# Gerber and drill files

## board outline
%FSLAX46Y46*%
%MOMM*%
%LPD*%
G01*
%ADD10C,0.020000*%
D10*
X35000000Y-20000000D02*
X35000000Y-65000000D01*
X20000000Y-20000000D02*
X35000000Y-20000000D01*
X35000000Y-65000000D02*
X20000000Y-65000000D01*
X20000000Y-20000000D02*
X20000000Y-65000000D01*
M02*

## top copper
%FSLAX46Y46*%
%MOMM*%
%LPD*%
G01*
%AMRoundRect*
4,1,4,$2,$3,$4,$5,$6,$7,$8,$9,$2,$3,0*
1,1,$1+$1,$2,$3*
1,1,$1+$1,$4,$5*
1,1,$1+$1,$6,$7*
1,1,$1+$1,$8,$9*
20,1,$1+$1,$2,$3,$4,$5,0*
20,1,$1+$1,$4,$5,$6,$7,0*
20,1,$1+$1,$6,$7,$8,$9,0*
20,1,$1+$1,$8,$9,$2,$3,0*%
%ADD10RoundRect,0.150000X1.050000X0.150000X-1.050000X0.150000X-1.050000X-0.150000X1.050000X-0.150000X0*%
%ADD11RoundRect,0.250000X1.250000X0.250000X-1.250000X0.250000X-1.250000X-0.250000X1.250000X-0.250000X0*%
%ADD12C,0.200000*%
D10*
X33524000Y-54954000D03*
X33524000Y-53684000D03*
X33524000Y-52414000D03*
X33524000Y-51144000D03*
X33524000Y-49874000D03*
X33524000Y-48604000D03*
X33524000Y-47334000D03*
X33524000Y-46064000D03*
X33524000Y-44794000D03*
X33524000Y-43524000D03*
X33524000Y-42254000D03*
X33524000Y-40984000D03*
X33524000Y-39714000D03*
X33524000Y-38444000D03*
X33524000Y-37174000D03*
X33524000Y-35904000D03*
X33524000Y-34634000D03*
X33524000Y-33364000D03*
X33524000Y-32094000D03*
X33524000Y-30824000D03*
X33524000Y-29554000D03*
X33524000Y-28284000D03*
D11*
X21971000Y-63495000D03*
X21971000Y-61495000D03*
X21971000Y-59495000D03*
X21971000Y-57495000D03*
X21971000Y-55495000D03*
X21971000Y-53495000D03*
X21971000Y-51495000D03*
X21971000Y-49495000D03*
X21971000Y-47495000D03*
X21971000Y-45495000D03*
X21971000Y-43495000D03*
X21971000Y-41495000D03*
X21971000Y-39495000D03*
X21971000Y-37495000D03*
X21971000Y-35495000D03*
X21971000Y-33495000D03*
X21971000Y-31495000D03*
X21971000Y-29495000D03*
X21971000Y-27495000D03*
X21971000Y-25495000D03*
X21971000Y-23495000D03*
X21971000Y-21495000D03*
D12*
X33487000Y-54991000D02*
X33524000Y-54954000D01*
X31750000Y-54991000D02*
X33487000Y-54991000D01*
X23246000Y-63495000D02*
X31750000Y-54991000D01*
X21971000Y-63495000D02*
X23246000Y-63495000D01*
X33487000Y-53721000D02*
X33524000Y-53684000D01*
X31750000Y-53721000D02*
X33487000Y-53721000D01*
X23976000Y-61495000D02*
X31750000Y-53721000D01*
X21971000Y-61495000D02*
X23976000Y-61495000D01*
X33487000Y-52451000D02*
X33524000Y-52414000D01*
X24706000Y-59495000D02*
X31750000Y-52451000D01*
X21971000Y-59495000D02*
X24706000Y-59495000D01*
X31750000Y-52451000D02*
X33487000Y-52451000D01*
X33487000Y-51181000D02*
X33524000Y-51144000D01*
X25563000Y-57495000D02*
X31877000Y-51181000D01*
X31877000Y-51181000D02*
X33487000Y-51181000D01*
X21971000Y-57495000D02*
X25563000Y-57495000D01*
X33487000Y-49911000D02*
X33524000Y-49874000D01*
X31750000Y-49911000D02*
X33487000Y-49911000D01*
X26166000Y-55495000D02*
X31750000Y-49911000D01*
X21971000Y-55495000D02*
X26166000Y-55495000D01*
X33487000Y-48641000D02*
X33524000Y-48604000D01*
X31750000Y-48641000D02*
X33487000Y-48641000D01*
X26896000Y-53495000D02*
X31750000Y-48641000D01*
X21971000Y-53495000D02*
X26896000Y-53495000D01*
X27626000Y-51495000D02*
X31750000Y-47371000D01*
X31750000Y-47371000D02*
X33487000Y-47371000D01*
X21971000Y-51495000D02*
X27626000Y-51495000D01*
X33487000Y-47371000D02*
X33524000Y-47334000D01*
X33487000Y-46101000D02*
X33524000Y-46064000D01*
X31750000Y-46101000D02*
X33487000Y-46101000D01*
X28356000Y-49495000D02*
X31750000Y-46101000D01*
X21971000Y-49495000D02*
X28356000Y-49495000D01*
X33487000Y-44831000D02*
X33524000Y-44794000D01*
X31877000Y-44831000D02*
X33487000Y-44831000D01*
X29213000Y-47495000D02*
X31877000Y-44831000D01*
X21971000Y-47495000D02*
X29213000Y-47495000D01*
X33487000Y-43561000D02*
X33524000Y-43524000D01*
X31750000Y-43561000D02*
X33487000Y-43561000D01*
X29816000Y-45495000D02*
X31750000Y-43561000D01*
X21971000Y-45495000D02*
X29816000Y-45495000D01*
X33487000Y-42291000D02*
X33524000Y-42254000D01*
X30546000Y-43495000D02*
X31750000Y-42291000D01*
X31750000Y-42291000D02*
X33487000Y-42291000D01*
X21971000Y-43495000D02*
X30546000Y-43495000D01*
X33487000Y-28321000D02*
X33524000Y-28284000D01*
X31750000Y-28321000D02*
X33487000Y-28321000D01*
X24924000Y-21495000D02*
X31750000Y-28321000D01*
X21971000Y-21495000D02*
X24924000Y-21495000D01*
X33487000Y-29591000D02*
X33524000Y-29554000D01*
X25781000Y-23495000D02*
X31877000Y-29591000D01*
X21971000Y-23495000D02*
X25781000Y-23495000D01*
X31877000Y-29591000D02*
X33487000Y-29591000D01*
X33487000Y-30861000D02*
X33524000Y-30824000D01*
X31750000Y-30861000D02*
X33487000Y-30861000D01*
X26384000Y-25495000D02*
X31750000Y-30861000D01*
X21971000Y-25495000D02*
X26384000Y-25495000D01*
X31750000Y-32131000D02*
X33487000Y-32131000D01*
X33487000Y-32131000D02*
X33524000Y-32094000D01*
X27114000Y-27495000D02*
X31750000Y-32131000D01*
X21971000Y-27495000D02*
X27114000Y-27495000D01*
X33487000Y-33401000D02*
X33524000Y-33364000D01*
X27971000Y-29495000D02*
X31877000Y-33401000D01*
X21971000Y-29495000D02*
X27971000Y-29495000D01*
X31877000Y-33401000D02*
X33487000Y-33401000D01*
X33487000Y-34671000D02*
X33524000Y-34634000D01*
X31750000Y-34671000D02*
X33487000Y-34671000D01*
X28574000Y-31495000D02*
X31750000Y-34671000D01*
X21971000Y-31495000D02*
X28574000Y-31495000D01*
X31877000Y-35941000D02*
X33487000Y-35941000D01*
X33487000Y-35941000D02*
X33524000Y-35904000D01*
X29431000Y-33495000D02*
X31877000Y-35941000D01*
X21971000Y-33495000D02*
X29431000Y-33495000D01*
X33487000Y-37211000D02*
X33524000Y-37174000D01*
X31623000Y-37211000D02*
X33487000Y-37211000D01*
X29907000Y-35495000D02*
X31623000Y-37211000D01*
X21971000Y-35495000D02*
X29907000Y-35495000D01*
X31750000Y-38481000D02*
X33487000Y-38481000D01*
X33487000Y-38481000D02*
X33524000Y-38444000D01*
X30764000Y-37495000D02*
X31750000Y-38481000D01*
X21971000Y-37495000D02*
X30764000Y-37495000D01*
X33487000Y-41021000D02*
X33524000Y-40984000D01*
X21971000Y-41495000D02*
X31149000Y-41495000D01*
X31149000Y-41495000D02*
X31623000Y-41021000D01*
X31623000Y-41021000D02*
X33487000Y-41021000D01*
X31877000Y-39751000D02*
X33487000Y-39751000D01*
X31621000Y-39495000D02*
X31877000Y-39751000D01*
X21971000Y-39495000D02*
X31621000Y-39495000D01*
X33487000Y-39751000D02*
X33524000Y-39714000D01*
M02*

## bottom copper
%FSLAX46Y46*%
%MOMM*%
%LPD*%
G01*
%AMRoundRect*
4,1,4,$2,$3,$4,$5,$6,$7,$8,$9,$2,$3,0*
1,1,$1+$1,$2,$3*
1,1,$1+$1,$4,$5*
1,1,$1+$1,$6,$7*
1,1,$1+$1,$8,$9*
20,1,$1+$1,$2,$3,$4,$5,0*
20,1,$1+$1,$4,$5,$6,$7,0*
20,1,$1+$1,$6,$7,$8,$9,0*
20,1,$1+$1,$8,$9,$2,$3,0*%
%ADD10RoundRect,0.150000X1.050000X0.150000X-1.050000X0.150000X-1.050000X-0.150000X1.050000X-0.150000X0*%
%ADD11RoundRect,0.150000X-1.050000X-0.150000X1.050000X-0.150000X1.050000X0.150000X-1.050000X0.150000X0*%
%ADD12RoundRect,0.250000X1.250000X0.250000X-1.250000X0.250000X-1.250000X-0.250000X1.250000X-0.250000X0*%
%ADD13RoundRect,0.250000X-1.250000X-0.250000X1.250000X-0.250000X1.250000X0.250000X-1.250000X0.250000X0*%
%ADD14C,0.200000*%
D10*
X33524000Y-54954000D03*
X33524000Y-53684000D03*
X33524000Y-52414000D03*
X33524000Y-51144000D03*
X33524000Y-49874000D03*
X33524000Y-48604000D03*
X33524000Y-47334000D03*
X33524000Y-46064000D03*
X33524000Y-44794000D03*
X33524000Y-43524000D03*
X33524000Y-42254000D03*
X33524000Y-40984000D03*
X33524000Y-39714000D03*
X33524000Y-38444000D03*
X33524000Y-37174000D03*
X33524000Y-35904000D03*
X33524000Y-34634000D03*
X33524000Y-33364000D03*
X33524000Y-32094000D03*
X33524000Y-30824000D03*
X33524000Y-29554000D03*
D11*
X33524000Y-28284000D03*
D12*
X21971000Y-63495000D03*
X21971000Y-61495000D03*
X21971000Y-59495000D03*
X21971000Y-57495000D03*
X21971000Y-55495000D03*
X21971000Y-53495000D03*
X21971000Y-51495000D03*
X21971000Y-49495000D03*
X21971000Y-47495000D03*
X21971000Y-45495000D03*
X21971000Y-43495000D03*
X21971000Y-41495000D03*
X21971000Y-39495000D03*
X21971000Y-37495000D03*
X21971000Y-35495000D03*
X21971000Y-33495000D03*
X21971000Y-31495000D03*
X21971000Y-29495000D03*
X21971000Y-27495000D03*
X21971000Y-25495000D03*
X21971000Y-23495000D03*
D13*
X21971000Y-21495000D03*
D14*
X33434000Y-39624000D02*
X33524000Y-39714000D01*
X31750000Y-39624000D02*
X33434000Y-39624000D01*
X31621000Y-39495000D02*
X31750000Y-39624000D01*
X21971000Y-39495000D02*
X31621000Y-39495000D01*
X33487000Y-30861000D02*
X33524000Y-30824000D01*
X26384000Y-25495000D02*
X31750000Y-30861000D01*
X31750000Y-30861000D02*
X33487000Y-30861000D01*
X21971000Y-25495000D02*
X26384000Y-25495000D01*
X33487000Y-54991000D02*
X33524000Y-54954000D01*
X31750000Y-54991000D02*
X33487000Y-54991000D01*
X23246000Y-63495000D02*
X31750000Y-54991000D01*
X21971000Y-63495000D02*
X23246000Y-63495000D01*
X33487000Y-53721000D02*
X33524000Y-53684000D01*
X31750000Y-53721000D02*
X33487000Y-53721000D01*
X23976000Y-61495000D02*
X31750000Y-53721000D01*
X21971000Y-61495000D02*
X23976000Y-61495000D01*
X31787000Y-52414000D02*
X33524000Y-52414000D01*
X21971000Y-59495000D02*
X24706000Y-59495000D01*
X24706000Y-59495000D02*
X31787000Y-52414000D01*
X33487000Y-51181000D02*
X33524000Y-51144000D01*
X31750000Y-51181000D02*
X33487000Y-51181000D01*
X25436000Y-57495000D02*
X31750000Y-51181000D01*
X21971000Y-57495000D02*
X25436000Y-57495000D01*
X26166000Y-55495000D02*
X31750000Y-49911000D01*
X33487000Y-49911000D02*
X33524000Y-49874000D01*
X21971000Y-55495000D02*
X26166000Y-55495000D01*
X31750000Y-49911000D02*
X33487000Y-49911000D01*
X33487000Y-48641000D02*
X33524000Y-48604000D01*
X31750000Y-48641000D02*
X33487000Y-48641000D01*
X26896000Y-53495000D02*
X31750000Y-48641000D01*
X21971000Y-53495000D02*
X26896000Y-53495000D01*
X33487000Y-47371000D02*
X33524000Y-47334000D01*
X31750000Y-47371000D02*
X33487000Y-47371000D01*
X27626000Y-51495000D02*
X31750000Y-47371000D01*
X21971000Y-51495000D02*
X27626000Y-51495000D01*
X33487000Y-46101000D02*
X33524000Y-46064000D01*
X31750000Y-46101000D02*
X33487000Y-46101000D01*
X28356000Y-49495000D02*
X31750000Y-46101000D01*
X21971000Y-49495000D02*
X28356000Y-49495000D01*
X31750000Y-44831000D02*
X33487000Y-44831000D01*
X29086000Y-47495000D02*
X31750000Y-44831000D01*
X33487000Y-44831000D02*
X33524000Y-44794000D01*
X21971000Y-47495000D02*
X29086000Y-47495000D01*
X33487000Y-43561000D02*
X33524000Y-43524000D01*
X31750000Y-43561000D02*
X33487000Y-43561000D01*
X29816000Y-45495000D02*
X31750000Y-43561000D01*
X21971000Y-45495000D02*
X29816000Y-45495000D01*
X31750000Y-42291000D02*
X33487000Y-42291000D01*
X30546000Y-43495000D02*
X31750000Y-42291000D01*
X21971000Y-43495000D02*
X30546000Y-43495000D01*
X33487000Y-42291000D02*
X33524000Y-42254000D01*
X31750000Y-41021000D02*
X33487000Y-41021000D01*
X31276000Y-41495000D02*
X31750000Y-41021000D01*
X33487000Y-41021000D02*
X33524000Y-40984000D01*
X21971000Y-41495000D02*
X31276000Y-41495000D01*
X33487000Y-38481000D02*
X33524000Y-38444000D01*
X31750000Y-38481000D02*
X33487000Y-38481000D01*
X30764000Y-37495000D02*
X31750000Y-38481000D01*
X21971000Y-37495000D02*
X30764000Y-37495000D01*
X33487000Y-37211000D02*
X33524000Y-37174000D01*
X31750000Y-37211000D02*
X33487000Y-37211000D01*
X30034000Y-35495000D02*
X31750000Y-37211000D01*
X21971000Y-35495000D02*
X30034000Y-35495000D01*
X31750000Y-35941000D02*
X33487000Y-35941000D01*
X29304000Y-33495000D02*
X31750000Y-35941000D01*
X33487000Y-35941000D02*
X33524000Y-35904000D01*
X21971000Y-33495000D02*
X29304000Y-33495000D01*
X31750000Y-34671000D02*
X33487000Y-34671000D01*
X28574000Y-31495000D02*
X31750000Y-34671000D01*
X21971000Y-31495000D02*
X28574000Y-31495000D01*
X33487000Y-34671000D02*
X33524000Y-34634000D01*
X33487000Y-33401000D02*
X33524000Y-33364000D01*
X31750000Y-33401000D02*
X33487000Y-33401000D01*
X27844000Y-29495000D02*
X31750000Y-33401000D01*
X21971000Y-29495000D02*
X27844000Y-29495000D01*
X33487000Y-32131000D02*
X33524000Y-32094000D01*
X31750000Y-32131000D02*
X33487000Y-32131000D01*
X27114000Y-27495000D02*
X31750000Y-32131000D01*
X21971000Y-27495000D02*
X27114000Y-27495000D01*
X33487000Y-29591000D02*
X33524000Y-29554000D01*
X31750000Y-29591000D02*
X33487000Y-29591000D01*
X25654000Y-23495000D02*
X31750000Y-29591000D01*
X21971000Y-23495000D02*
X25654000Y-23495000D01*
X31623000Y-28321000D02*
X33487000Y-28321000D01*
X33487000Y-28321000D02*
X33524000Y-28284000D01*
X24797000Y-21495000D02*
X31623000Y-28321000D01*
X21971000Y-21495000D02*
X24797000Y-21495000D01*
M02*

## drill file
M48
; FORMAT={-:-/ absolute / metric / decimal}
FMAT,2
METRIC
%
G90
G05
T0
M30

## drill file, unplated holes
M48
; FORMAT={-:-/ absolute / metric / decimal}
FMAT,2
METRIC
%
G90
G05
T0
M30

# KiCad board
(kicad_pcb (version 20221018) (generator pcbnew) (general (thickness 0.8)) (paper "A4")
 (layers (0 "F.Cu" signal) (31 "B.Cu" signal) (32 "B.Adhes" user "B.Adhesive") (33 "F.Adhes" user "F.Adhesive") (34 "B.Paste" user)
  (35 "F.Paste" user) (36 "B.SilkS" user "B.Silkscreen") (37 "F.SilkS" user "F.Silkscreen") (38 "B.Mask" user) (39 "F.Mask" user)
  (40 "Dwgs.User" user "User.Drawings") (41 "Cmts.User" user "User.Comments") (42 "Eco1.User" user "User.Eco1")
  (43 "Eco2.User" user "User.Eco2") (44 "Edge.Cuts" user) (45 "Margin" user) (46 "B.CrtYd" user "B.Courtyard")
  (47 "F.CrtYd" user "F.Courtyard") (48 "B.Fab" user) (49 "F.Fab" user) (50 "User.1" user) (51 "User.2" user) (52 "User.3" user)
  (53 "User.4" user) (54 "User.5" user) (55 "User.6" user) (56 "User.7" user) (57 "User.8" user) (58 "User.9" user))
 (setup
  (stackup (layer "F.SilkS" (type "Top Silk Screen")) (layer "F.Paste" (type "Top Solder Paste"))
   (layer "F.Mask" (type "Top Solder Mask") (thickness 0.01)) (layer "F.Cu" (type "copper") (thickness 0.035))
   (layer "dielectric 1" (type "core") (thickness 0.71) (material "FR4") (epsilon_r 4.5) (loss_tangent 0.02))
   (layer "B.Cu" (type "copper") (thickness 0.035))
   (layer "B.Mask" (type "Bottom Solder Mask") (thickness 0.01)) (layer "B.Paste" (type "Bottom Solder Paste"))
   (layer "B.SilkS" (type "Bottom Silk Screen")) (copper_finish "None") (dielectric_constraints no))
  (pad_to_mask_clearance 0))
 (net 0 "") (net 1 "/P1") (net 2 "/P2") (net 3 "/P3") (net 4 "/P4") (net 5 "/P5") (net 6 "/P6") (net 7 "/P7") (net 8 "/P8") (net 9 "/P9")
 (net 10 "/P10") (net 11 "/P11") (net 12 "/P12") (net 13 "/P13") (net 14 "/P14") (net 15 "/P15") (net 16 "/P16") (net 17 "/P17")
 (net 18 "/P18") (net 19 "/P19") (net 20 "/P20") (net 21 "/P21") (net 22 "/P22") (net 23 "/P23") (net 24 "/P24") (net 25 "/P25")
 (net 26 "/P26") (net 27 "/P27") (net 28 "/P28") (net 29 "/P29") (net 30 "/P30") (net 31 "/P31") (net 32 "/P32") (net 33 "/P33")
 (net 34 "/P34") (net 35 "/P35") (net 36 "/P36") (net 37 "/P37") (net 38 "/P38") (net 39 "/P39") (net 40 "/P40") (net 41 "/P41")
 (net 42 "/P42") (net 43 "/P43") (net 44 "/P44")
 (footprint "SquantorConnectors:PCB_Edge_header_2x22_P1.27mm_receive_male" (layer "F.Cu") (at 28.524 41.619 -90)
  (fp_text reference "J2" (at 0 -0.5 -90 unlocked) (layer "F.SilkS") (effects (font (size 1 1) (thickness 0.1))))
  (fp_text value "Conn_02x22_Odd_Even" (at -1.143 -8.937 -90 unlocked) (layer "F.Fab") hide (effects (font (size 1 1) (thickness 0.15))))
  (pad "1" smd roundrect (at 13.335 -5 180) (size 2.4 0.6) (layers "B.Cu" "B.Paste" "B.Mask") (roundrect_rratio 0.25) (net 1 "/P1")
   (thermal_bridge_angle 45))
  (pad "2" smd roundrect (at 13.335 -5 180) (size 2.4 0.6) (layers "F.Cu" "F.Paste" "F.Mask") (roundrect_rratio 0.25) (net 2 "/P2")
   (thermal_bridge_angle 45))
  (pad "3" smd roundrect (at 12.065 -5 180) (size 2.4 0.6) (layers "B.Cu" "B.Paste" "B.Mask") (roundrect_rratio 0.25) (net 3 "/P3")
   (thermal_bridge_angle 45))
  (pad "4" smd roundrect (at 12.065 -5 180) (size 2.4 0.6) (layers "F.Cu" "F.Paste" "F.Mask") (roundrect_rratio 0.25) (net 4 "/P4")
   (thermal_bridge_angle 45))
  (pad "5" smd roundrect (at 10.795 -5 180) (size 2.4 0.6) (layers "B.Cu" "B.Paste" "B.Mask") (roundrect_rratio 0.25) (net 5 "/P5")
   (thermal_bridge_angle 45))
  (pad "6" smd roundrect (at 10.795 -5 180) (size 2.4 0.6) (layers "F.Cu" "F.Paste" "F.Mask") (roundrect_rratio 0.25) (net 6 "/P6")
   (thermal_bridge_angle 45))
  (pad "7" smd roundrect (at 9.525 -5 180) (size 2.4 0.6) (layers "B.Cu" "B.Paste" "B.Mask") (roundrect_rratio 0.25) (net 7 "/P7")
   (thermal_bridge_angle 45))
  (pad "8" smd roundrect (at 9.525 -5 180) (size 2.4 0.6) (layers "F.Cu" "F.Paste" "F.Mask") (roundrect_rratio 0.25) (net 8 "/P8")
   (thermal_bridge_angle 45))
  (pad "9" smd roundrect (at 8.255 -5 180) (size 2.4 0.6) (layers "B.Cu" "B.Paste" "B.Mask") (roundrect_rratio 0.25) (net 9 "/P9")
   (thermal_bridge_angle 45))
  (pad "10" smd roundrect (at 8.255 -5 180) (size 2.4 0.6) (layers "F.Cu" "F.Paste" "F.Mask") (roundrect_rratio 0.25) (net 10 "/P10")
   (thermal_bridge_angle 45))
  (pad "11" smd roundrect (at 6.985 -5 180) (size 2.4 0.6) (layers "B.Cu" "B.Paste" "B.Mask") (roundrect_rratio 0.25) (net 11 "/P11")
   (thermal_bridge_angle 45))
  (pad "12" smd roundrect (at 6.985 -5 180) (size 2.4 0.6) (layers "F.Cu" "F.Paste" "F.Mask") (roundrect_rratio 0.25) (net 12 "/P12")
   (thermal_bridge_angle 45))
  (pad "13" smd roundrect (at 5.715 -5 180) (size 2.4 0.6) (layers "B.Cu" "B.Paste" "B.Mask") (roundrect_rratio 0.25) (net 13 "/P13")
   (thermal_bridge_angle 45))
  (pad "14" smd roundrect (at 5.715 -5 180) (size 2.4 0.6) (layers "F.Cu" "F.Paste" "F.Mask") (roundrect_rratio 0.25) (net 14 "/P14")
   (thermal_bridge_angle 45))
  (pad "15" smd roundrect (at 4.445 -5 180) (size 2.4 0.6) (layers "B.Cu" "B.Paste" "B.Mask") (roundrect_rratio 0.25) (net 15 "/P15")
   (thermal_bridge_angle 45))
  (pad "16" smd roundrect (at 4.445 -5 180) (size 2.4 0.6) (layers "F.Cu" "F.Paste" "F.Mask") (roundrect_rratio 0.25) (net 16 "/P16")
   (thermal_bridge_angle 45))
  (pad "17" smd roundrect (at 3.175 -5 180) (size 2.4 0.6) (layers "B.Cu" "B.Paste" "B.Mask") (roundrect_rratio 0.25) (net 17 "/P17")
   (thermal_bridge_angle 45))
  (pad "18" smd roundrect (at 3.175 -5 180) (size 2.4 0.6) (layers "F.Cu" "F.Paste" "F.Mask") (roundrect_rratio 0.25) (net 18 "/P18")
   (thermal_bridge_angle 45))
  (pad "19" smd roundrect (at 1.905 -5 180) (size 2.4 0.6) (layers "B.Cu" "B.Paste" "B.Mask") (roundrect_rratio 0.25) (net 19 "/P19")
   (thermal_bridge_angle 45))
  (pad "20" smd roundrect (at 1.905 -5 180) (size 2.4 0.6) (layers "F.Cu" "F.Paste" "F.Mask") (roundrect_rratio 0.25) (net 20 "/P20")
   (thermal_bridge_angle 45))
  (pad "21" smd roundrect (at 0.635 -5 180) (size 2.4 0.6) (layers "B.Cu" "B.Paste" "B.Mask") (roundrect_rratio 0.25) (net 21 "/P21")
   (thermal_bridge_angle 45))
  (pad "22" smd roundrect (at 0.635 -5 180) (size 2.4 0.6) (layers "F.Cu" "F.Paste" "F.Mask") (roundrect_rratio 0.25) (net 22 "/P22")
   (thermal_bridge_angle 45))
  (pad "23" smd roundrect (at -0.635 -5 180) (size 2.4 0.6) (layers "B.Cu" "B.Paste" "B.Mask") (roundrect_rratio 0.25) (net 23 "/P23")
   (thermal_bridge_angle 45))
  (pad "24" smd roundrect (at -0.635 -5 180) (size 2.4 0.6) (layers "F.Cu" "F.Paste" "F.Mask") (roundrect_rratio 0.25) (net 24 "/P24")
   (thermal_bridge_angle 45))
  (pad "25" smd roundrect (at -1.905 -5 180) (size 2.4 0.6) (layers "B.Cu" "B.Paste" "B.Mask") (roundrect_rratio 0.25) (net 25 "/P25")
   (thermal_bridge_angle 45))
  (pad "26" smd roundrect (at -1.905 -5 180) (size 2.4 0.6) (layers "F.Cu" "F.Paste" "F.Mask") (roundrect_rratio 0.25) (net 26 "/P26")
   (thermal_bridge_angle 45))
  (pad "27" smd roundrect (at -3.175 -5 180) (size 2.4 0.6) (layers "B.Cu" "B.Paste" "B.Mask") (roundrect_rratio 0.25) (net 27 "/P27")
   (thermal_bridge_angle 45))
  (pad "28" smd roundrect (at -3.175 -5 180) (size 2.4 0.6) (layers "F.Cu" "F.Paste" "F.Mask") (roundrect_rratio 0.25) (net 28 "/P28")
   (thermal_bridge_angle 45))
  (pad "29" smd roundrect (at -4.445 -5 180) (size 2.4 0.6) (layers "B.Cu" "B.Paste" "B.Mask") (roundrect_rratio 0.25) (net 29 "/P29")
   (thermal_bridge_angle 45))
  (pad "30" smd roundrect (at -4.445 -5 180) (size 2.4 0.6) (layers "F.Cu" "F.Paste" "F.Mask") (roundrect_rratio 0.25) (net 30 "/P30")
   (thermal_bridge_angle 45))
  (pad "31" smd roundrect (at -5.715 -5 180) (size 2.4 0.6) (layers "B.Cu" "B.Paste" "B.Mask") (roundrect_rratio 0.25) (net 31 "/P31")
   (thermal_bridge_angle 45))
  (pad "32" smd roundrect (at -5.715 -5 180) (size 2.4 0.6) (layers "F.Cu" "F.Paste" "F.Mask") (roundrect_rratio 0.25) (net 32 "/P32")
   (thermal_bridge_angle 45))
  (pad "33" smd roundrect (at -6.985 -5 180) (size 2.4 0.6) (layers "B.Cu" "B.Paste" "B.Mask") (roundrect_rratio 0.25) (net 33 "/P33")
   (thermal_bridge_angle 45))
  (pad "34" smd roundrect (at -6.985 -5 180) (size 2.4 0.6) (layers "F.Cu" "F.Paste" "F.Mask") (roundrect_rratio 0.25) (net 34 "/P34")
   (thermal_bridge_angle 45))
  (pad "35" smd roundrect (at -8.255 -5 180) (size 2.4 0.6) (layers "B.Cu" "B.Paste" "B.Mask") (roundrect_rratio 0.25) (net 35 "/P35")
   (thermal_bridge_angle 45))
  (pad "36" smd roundrect (at -8.255 -5 180) (size 2.4 0.6) (layers "F.Cu" "F.Paste" "F.Mask") (roundrect_rratio 0.25) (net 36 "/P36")
   (thermal_bridge_angle 45))
  (pad "37" smd roundrect (at -9.525 -5 180) (size 2.4 0.6) (layers "B.Cu" "B.Paste" "B.Mask") (roundrect_rratio 0.25) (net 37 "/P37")
   (thermal_bridge_angle 45))
  (pad "38" smd roundrect (at -9.525 -5 180) (size 2.4 0.6) (layers "F.Cu" "F.Paste" "F.Mask") (roundrect_rratio 0.25) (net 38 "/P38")
   (thermal_bridge_angle 45))
  (pad "39" smd roundrect (at -10.795 -5 180) (size 2.4 0.6) (layers "B.Cu" "B.Paste" "B.Mask") (roundrect_rratio 0.25) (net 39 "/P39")
   (thermal_bridge_angle 45))
  (pad "40" smd roundrect (at -10.795 -5 180) (size 2.4 0.6) (layers "F.Cu" "F.Paste" "F.Mask") (roundrect_rratio 0.25) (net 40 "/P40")
   (thermal_bridge_angle 45))
  (pad "41" smd roundrect (at -12.065 -5 180) (size 2.4 0.6) (layers "B.Cu" "B.Paste" "B.Mask") (roundrect_rratio 0.25) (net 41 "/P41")
   (thermal_bridge_angle 45))
  (pad "42" smd roundrect (at -12.065 -5 180) (size 2.4 0.6) (layers "F.Cu" "F.Paste" "F.Mask") (roundrect_rratio 0.25) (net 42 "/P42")
   (thermal_bridge_angle 45))
  (pad "43" smd roundrect (at -13.335 -5) (size 2.4 0.6) (layers "B.Cu" "B.Paste" "B.Mask") (roundrect_rratio 0.25) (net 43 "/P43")
   (thermal_bridge_angle 45))
  (pad "44" smd roundrect (at -13.335 -5 180) (size 2.4 0.6) (layers "F.Cu" "F.Paste" "F.Mask") (roundrect_rratio 0.25) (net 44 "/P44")
   (thermal_bridge_angle 45)))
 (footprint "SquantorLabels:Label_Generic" (layer "F.Cu") (at 24.892 26.0745 90)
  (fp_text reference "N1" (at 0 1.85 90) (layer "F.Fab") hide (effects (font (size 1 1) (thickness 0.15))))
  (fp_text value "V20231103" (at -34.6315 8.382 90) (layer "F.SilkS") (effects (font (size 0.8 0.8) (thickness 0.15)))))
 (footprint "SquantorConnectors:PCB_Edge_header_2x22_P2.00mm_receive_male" (layer "F.Cu") (at 16.971 42.495 -90)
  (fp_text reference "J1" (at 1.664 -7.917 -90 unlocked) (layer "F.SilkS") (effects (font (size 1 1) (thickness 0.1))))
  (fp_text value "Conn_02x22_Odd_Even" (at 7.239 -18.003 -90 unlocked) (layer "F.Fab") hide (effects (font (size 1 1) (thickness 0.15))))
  (pad "1" smd roundrect (at 21 -5 180) (size 3 1) (layers "B.Cu" "B.Paste" "B.Mask") (roundrect_rratio 0.25) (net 1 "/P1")
   (thermal_bridge_angle 45))
  (pad "2" smd roundrect (at 21 -5 180) (size 3 1) (layers "F.Cu" "F.Paste" "F.Mask") (roundrect_rratio 0.25) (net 2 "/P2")
   (thermal_bridge_angle 45))
  (pad "3" smd roundrect (at 19 -5 180) (size 3 1) (layers "B.Cu" "B.Paste" "B.Mask") (roundrect_rratio 0.25) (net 3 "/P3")
   (thermal_bridge_angle 45))
  (pad "4" smd roundrect (at 19 -5 180) (size 3 1) (layers "F.Cu" "F.Paste" "F.Mask") (roundrect_rratio 0.25) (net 4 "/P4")
   (thermal_bridge_angle 45))
  (pad "5" smd roundrect (at 17 -5 180) (size 3 1) (layers "B.Cu" "B.Paste" "B.Mask") (roundrect_rratio 0.25) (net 5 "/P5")
   (thermal_bridge_angle 45))
  (pad "6" smd roundrect (at 17 -5 180) (size 3 1) (layers "F.Cu" "F.Paste" "F.Mask") (roundrect_rratio 0.25) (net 6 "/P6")
   (thermal_bridge_angle 45))
  (pad "7" smd roundrect (at 15 -5 180) (size 3 1) (layers "B.Cu" "B.Paste" "B.Mask") (roundrect_rratio 0.25) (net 7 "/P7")
   (thermal_bridge_angle 45))
  (pad "8" smd roundrect (at 15 -5 180) (size 3 1) (layers "F.Cu" "F.Paste" "F.Mask") (roundrect_rratio 0.25) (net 8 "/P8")
   (thermal_bridge_angle 45))
  (pad "9" smd roundrect (at 13 -5 180) (size 3 1) (layers "B.Cu" "B.Paste" "B.Mask") (roundrect_rratio 0.25) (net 9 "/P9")
   (thermal_bridge_angle 45))
  (pad "10" smd roundrect (at 13 -5 180) (size 3 1) (layers "F.Cu" "F.Paste" "F.Mask") (roundrect_rratio 0.25) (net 10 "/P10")
   (thermal_bridge_angle 45))
  (pad "11" smd roundrect (at 11 -5 180) (size 3 1) (layers "B.Cu" "B.Paste" "B.Mask") (roundrect_rratio 0.25) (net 11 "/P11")
   (thermal_bridge_angle 45))
  (pad "12" smd roundrect (at 11 -5 180) (size 3 1) (layers "F.Cu" "F.Paste" "F.Mask") (roundrect_rratio 0.25) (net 12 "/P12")
   (thermal_bridge_angle 45))
  (pad "13" smd roundrect (at 9 -5 180) (size 3 1) (layers "B.Cu" "B.Paste" "B.Mask") (roundrect_rratio 0.25) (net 13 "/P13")
   (thermal_bridge_angle 45))
  (pad "14" smd roundrect (at 9 -5 180) (size 3 1) (layers "F.Cu" "F.Paste" "F.Mask") (roundrect_rratio 0.25) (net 14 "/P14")
   (thermal_bridge_angle 45))
  (pad "15" smd roundrect (at 7 -5 180) (size 3 1) (layers "B.Cu" "B.Paste" "B.Mask") (roundrect_rratio 0.25) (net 15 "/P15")
   (thermal_bridge_angle 45))
  (pad "16" smd roundrect (at 7 -5 180) (size 3 1) (layers "F.Cu" "F.Paste" "F.Mask") (roundrect_rratio 0.25) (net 16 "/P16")
   (thermal_bridge_angle 45))
  (pad "17" smd roundrect (at 5 -5 180) (size 3 1) (layers "B.Cu" "B.Paste" "B.Mask") (roundrect_rratio 0.25) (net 17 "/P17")
   (thermal_bridge_angle 45))
  (pad "18" smd roundrect (at 5 -5 180) (size 3 1) (layers "F.Cu" "F.Paste" "F.Mask") (roundrect_rratio 0.25) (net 18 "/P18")
   (thermal_bridge_angle 45))
  (pad "19" smd roundrect (at 3 -5 180) (size 3 1) (layers "B.Cu" "B.Paste" "B.Mask") (roundrect_rratio 0.25) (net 19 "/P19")
   (thermal_bridge_angle 45))
  (pad "20" smd roundrect (at 3 -5 180) (size 3 1) (layers "F.Cu" "F.Paste" "F.Mask") (roundrect_rratio 0.25) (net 20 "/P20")
   (thermal_bridge_angle 45))
  (pad "21" smd roundrect (at 1 -5 180) (size 3 1) (layers "B.Cu" "B.Paste" "B.Mask") (roundrect_rratio 0.25) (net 21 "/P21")
   (thermal_bridge_angle 45))
  (pad "22" smd roundrect (at 1 -5 180) (size 3 1) (layers "F.Cu" "F.Paste" "F.Mask") (roundrect_rratio 0.25) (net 22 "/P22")
   (thermal_bridge_angle 45))
  (pad "23" smd roundrect (at -1 -5 180) (size 3 1) (layers "B.Cu" "B.Paste" "B.Mask") (roundrect_rratio 0.25) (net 23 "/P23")
   (thermal_bridge_angle 45))
  (pad "24" smd roundrect (at -1 -5 180) (size 3 1) (layers "F.Cu" "F.Paste" "F.Mask") (roundrect_rratio 0.25) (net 24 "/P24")
   (thermal_bridge_angle 45))
  (pad "25" smd roundrect (at -3 -5 180) (size 3 1) (layers "B.Cu" "B.Paste" "B.Mask") (roundrect_rratio 0.25) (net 25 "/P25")
   (thermal_bridge_angle 45))
  (pad "26" smd roundrect (at -3 -5 180) (size 3 1) (layers "F.Cu" "F.Paste" "F.Mask") (roundrect_rratio 0.25) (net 26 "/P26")
   (thermal_bridge_angle 45))
  (pad "27" smd roundrect (at -5 -5 180) (size 3 1) (layers "B.Cu" "B.Paste" "B.Mask") (roundrect_rratio 0.25) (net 27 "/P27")
   (thermal_bridge_angle 45))
  (pad "28" smd roundrect (at -5 -5 180) (size 3 1) (layers "F.Cu" "F.Paste" "F.Mask") (roundrect_rratio 0.25) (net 28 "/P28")
   (thermal_bridge_angle 45))
  (pad "29" smd roundrect (at -7 -5 180) (size 3 1) (layers "B.Cu" "B.Paste" "B.Mask") (roundrect_rratio 0.25) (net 29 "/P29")
   (thermal_bridge_angle 45))
  (pad "30" smd roundrect (at -7 -5 180) (size 3 1) (layers "F.Cu" "F.Paste" "F.Mask") (roundrect_rratio 0.25) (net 30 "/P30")
   (thermal_bridge_angle 45))
  (pad "31" smd roundrect (at -9 -5 180) (size 3 1) (layers "B.Cu" "B.Paste" "B.Mask") (roundrect_rratio 0.25) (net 31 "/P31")
   (thermal_bridge_angle 45))
  (pad "32" smd roundrect (at -9 -5 180) (size 3 1) (layers "F.Cu" "F.Paste" "F.Mask") (roundrect_rratio 0.25) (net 32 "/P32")
   (thermal_bridge_angle 45))
  (pad "33" smd roundrect (at -11 -5 180) (size 3 1) (layers "B.Cu" "B.Paste" "B.Mask") (roundrect_rratio 0.25) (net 33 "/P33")
   (thermal_bridge_angle 45))
  (pad "34" smd roundrect (at -11 -5 180) (size 3 1) (layers "F.Cu" "F.Paste" "F.Mask") (roundrect_rratio 0.25) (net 34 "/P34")
   (thermal_bridge_angle 45))
  (pad "35" smd roundrect (at -13 -5 180) (size 3 1) (layers "B.Cu" "B.Paste" "B.Mask") (roundrect_rratio 0.25) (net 35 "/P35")
   (thermal_bridge_angle 45))
  (pad "36" smd roundrect (at -13 -5 180) (size 3 1) (layers "F.Cu" "F.Paste" "F.Mask") (roundrect_rratio 0.25) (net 36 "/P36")
   (thermal_bridge_angle 45))
  (pad "37" smd roundrect (at -15 -5 180) (size 3 1) (layers "B.Cu" "B.Paste" "B.Mask") (roundrect_rratio 0.25) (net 37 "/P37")
   (thermal_bridge_angle 45))
  (pad "38" smd roundrect (at -15 -5 180) (size 3 1) (layers "F.Cu" "F.Paste" "F.Mask") (roundrect_rratio 0.25) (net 38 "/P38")
   (thermal_bridge_angle 45))
  (pad "39" smd roundrect (at -17 -5 180) (size 3 1) (layers "B.Cu" "B.Paste" "B.Mask") (roundrect_rratio 0.25) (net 39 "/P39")
   (thermal_bridge_angle 45))
  (pad "40" smd roundrect (at -17 -5 180) (size 3 1) (layers "F.Cu" "F.Paste" "F.Mask") (roundrect_rratio 0.25) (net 40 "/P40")
   (thermal_bridge_angle 45))
  (pad "41" smd roundrect (at -19 -5 180) (size 3 1) (layers "B.Cu" "B.Paste" "B.Mask") (roundrect_rratio 0.25) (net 41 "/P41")
   (thermal_bridge_angle 45))
  (pad "42" smd roundrect (at -19 -5 180) (size 3 1) (layers "F.Cu" "F.Paste" "F.Mask") (roundrect_rratio 0.25) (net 42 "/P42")
   (thermal_bridge_angle 45))
  (pad "43" smd roundrect (at -21 -5) (size 3 1) (layers "B.Cu" "B.Paste" "B.Mask") (roundrect_rratio 0.25) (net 43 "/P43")
   (thermal_bridge_angle 45))
  (pad "44" smd roundrect (at -21 -5 180) (size 3 1) (layers "F.Cu" "F.Paste" "F.Mask") (roundrect_rratio 0.25) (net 44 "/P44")
   (thermal_bridge_angle 45)))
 (gr_line (start 35 20) (end 35 65) (stroke (width 0.02) (type solid)) (layer "Edge.Cuts"))
 (gr_line (start 20 20) (end 35 20) (stroke (width 0.02) (type solid)) (layer "Edge.Cuts"))
 (gr_line (start 35 65) (end 20 65) (stroke (width 0.02) (type solid)) (layer "Edge.Cuts"))
 (gr_line (start 20 20) (end 20 65) (stroke (width 0.02) (type solid)) (layer "Edge.Cuts"))
 (segment (start 23.246 63.495) (end 31.75 54.991) (width 0.2) (layer "B.Cu") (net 1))
 (segment (start 31.75 54.991) (end 33.487 54.991) (width 0.2) (layer "B.Cu") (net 1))
 (segment (start 21.971 63.495) (end 23.246 63.495) (width 0.2) (layer "B.Cu") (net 1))
 (segment (start 33.487 54.991) (end 33.524 54.954) (width 0.2) (layer "B.Cu") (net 1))
 (segment (start 33.487 54.991) (end 33.524 54.954) (width 0.2) (layer "F.Cu") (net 2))
 (segment (start 23.246 63.495) (end 31.75 54.991) (width 0.2) (layer "F.Cu") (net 2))
 (segment (start 31.75 54.991) (end 33.487 54.991) (width 0.2) (layer "F.Cu") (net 2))
 (segment (start 21.971 63.495) (end 23.246 63.495) (width 0.2) (layer "F.Cu") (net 2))
 (segment (start 23.976 61.495) (end 31.75 53.721) (width 0.2) (layer "B.Cu") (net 3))
 (segment (start 33.487 53.721) (end 33.524 53.684) (width 0.2) (layer "B.Cu") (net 3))
 (segment (start 31.75 53.721) (end 33.487 53.721) (width 0.2) (layer "B.Cu") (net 3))
 (segment (start 21.971 61.495) (end 23.976 61.495) (width 0.2) (layer "B.Cu") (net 3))
 (segment (start 33.487 53.721) (end 33.524 53.684) (width 0.2) (layer "F.Cu") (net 4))
 (segment (start 23.976 61.495) (end 31.75 53.721) (width 0.2) (layer "F.Cu") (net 4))
 (segment (start 31.75 53.721) (end 33.487 53.721) (width 0.2) (layer "F.Cu") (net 4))
 (segment (start 21.971 61.495) (end 23.976 61.495) (width 0.2) (layer "F.Cu") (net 4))
 (segment (start 21.971 59.495) (end 24.706 59.495) (width 0.2) (layer "B.Cu") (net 5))
 (segment (start 24.706 59.495) (end 31.787 52.414) (width 0.2) (layer "B.Cu") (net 5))
 (segment (start 31.787 52.414) (end 33.524 52.414) (width 0.2) (layer "B.Cu") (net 5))
 (segment (start 21.971 59.495) (end 24.706 59.495) (width 0.2) (layer "F.Cu") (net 6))
 (segment (start 31.75 52.451) (end 33.487 52.451) (width 0.2) (layer "F.Cu") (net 6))
 (segment (start 24.706 59.495) (end 31.75 52.451) (width 0.2) (layer "F.Cu") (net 6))
 (segment (start 33.487 52.451) (end 33.524 52.414) (width 0.2) (layer "F.Cu") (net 6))
 (segment (start 25.436 57.495) (end 31.75 51.181) (width 0.2) (layer "B.Cu") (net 7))
 (segment (start 31.75 51.181) (end 33.487 51.181) (width 0.2) (layer "B.Cu") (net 7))
 (segment (start 21.971 57.495) (end 25.436 57.495) (width 0.2) (layer "B.Cu") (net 7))
 (segment (start 33.487 51.181) (end 33.524 51.144) (width 0.2) (layer "B.Cu") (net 7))
 (segment (start 21.971 57.495) (end 25.563 57.495) (width 0.2) (layer "F.Cu") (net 8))
 (segment (start 33.487 51.181) (end 33.524 51.144) (width 0.2) (layer "F.Cu") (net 8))
 (segment (start 31.877 51.181) (end 33.487 51.181) (width 0.2) (layer "F.Cu") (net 8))
 (segment (start 25.563 57.495) (end 31.877 51.181) (width 0.2) (layer "F.Cu") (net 8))
 (segment (start 31.75 49.911) (end 33.487 49.911) (width 0.2) (layer "B.Cu") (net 9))
 (segment (start 21.971 55.495) (end 26.166 55.495) (width 0.2) (layer "B.Cu") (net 9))
 (segment (start 26.166 55.495) (end 31.75 49.911) (width 0.2) (layer "B.Cu") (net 9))
 (segment (start 33.487 49.911) (end 33.524 49.874) (width 0.2) (layer "B.Cu") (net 9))
 (segment (start 21.971 55.495) (end 26.166 55.495) (width 0.2) (layer "F.Cu") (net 10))
 (segment (start 33.487 49.911) (end 33.524 49.874) (width 0.2) (layer "F.Cu") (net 10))
 (segment (start 26.166 55.495) (end 31.75 49.911) (width 0.2) (layer "F.Cu") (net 10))
 (segment (start 31.75 49.911) (end 33.487 49.911) (width 0.2) (layer "F.Cu") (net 10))
 (segment (start 31.75 48.641) (end 33.487 48.641) (width 0.2) (layer "B.Cu") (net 11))
 (segment (start 26.896 53.495) (end 31.75 48.641) (width 0.2) (layer "B.Cu") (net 11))
 (segment (start 33.487 48.641) (end 33.524 48.604) (width 0.2) (layer "B.Cu") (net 11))
 (segment (start 21.971 53.495) (end 26.896 53.495) (width 0.2) (layer "B.Cu") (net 11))
 (segment (start 21.971 53.495) (end 26.896 53.495) (width 0.2) (layer "F.Cu") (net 12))
 (segment (start 26.896 53.495) (end 31.75 48.641) (width 0.2) (layer "F.Cu") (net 12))
 (segment (start 31.75 48.641) (end 33.487 48.641) (width 0.2) (layer "F.Cu") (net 12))
 (segment (start 33.487 48.641) (end 33.524 48.604) (width 0.2) (layer "F.Cu") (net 12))
 (segment (start 33.487 47.371) (end 33.524 47.334) (width 0.2) (layer "B.Cu") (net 13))
 (segment (start 27.626 51.495) (end 31.75 47.371) (width 0.2) (layer "B.Cu") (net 13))
 (segment (start 31.75 47.371) (end 33.487 47.371) (width 0.2) (layer "B.Cu") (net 13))
 (segment (start 21.971 51.495) (end 27.626 51.495) (width 0.2) (layer "B.Cu") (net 13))
 (segment (start 33.487 47.371) (end 33.524 47.334) (width 0.2) (layer "F.Cu") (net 14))
 (segment (start 21.971 51.495) (end 27.626 51.495) (width 0.2) (layer "F.Cu") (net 14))
 (segment (start 27.626 51.495) (end 31.75 47.371) (width 0.2) (layer "F.Cu") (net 14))
 (segment (start 31.75 47.371) (end 33.487 47.371) (width 0.2) (layer "F.Cu") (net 14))
 (segment (start 28.356 49.495) (end 31.75 46.101) (width 0.2) (layer "B.Cu") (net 15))
 (segment (start 21.971 49.495) (end 28.356 49.495) (width 0.2) (layer "B.Cu") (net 15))
 (segment (start 33.487 46.101) (end 33.524 46.064) (width 0.2) (layer "B.Cu") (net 15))
 (segment (start 31.75 46.101) (end 33.487 46.101) (width 0.2) (layer "B.Cu") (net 15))
 (segment (start 33.487 46.101) (end 33.524 46.064) (width 0.2) (layer "F.Cu") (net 16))
 (segment (start 28.356 49.495) (end 31.75 46.101) (width 0.2) (layer "F.Cu") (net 16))
 (segment (start 31.75 46.101) (end 33.487 46.101) (width 0.2) (layer "F.Cu") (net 16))
 (segment (start 21.971 49.495) (end 28.356 49.495) (width 0.2) (layer "F.Cu") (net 16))
 (segment (start 33.487 44.831) (end 33.524 44.794) (width 0.2) (layer "B.Cu") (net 17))
 (segment (start 29.086 47.495) (end 31.75 44.831) (width 0.2) (layer "B.Cu") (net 17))
 (segment (start 31.75 44.831) (end 33.487 44.831) (width 0.2) (layer "B.Cu") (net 17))
 (segment (start 21.971 47.495) (end 29.086 47.495) (width 0.2) (layer "B.Cu") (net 17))
 (segment (start 21.971 47.495) (end 29.213 47.495) (width 0.2) (layer "F.Cu") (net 18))
 (segment (start 33.487 44.831) (end 33.524 44.794) (width 0.2) (layer "F.Cu") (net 18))
 (segment (start 31.877 44.831) (end 33.487 44.831) (width 0.2) (layer "F.Cu") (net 18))
 (segment (start 29.213 47.495) (end 31.877 44.831) (width 0.2) (layer "F.Cu") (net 18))
 (segment (start 33.487 43.561) (end 33.524 43.524) (width 0.2) (layer "B.Cu") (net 19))
 (segment (start 29.816 45.495) (end 31.75 43.561) (width 0.2) (layer "B.Cu") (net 19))
 (segment (start 21.971 45.495) (end 29.816 45.495) (width 0.2) (layer "B.Cu") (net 19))
 (segment (start 31.75 43.561) (end 33.487 43.561) (width 0.2) (layer "B.Cu") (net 19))
 (segment (start 33.487 43.561) (end 33.524 43.524) (width 0.2) (layer "F.Cu") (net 20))
 (segment (start 31.75 43.561) (end 33.487 43.561) (width 0.2) (layer "F.Cu") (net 20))
 (segment (start 29.816 45.495) (end 31.75 43.561) (width 0.2) (layer "F.Cu") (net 20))
 (segment (start 21.971 45.495) (end 29.816 45.495) (width 0.2) (layer "F.Cu") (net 20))
 (segment (start 33.487 42.291) (end 33.524 42.254) (width 0.2) (layer "B.Cu") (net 21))
 (segment (start 30.546 43.495) (end 31.75 42.291) (width 0.2) (layer "B.Cu") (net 21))
 (segment (start 31.75 42.291) (end 33.487 42.291) (width 0.2) (layer "B.Cu") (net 21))
 (segment (start 21.971 43.495) (end 30.546 43.495) (width 0.2) (layer "B.Cu") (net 21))
 (segment (start 33.487 42.291) (end 33.524 42.254) (width 0.2) (layer "F.Cu") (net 22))
 (segment (start 21.971 43.495) (end 30.546 43.495) (width 0.2) (layer "F.Cu") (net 22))
 (segment (start 30.546 43.495) (end 31.75 42.291) (width 0.2) (layer "F.Cu") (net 22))
 (segment (start 31.75 42.291) (end 33.487 42.291) (width 0.2) (layer "F.Cu") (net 22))
 (segment (start 33.487 41.021) (end 33.524 40.984) (width 0.2) (layer "B.Cu") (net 23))
 (segment (start 31.75 41.021) (end 33.487 41.021) (width 0.2) (layer "B.Cu") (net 23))
 (segment (start 31.276 41.495) (end 31.75 41.021) (width 0.2) (layer "B.Cu") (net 23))
 (segment (start 21.971 41.495) (end 31.276 41.495) (width 0.2) (layer "B.Cu") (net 23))
 (segment (start 33.487 41.021) (end 33.524 40.984) (width 0.2) (layer "F.Cu") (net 24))
 (segment (start 21.971 41.495) (end 31.149 41.495) (width 0.2) (layer "F.Cu") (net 24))
 (segment (start 31.149 41.495) (end 31.623 41.021) (width 0.2) (layer "F.Cu") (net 24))
 (segment (start 31.623 41.021) (end 33.487 41.021) (width 0.2) (layer "F.Cu") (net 24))
 (segment (start 21.971 39.495) (end 31.621 39.495) (width 0.2) (layer "B.Cu") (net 25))
 (segment (start 31.75 39.624) (end 33.434 39.624) (width 0.2) (layer "B.Cu") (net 25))
 (segment (start 31.621 39.495) (end 31.75 39.624) (width 0.2) (layer "B.Cu") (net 25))
 (segment (start 33.434 39.624) (end 33.524 39.714) (width 0.2) (layer "B.Cu") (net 25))
 (segment (start 31.877 39.751) (end 33.487 39.751) (width 0.2) (layer "F.Cu") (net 26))
 (segment (start 31.621 39.495) (end 31.877 39.751) (width 0.2) (layer "F.Cu") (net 26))
 (segment (start 21.971 39.495) (end 31.621 39.495) (width 0.2) (layer "F.Cu") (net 26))
 (segment (start 33.487 39.751) (end 33.524 39.714) (width 0.2) (layer "F.Cu") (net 26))
 (segment (start 30.764 37.495) (end 31.75 38.481) (width 0.2) (layer "B.Cu") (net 27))
 (segment (start 33.487 38.481) (end 33.524 38.444) (width 0.2) (layer "B.Cu") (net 27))
 (segment (start 31.75 38.481) (end 33.487 38.481) (width 0.2) (layer "B.Cu") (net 27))
 (segment (start 21.971 37.495) (end 30.764 37.495) (width 0.2) (layer "B.Cu") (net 27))
 (segment (start 30.764 37.495) (end 31.75 38.481) (width 0.2) (layer "F.Cu") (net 28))
 (segment (start 33.487 38.481) (end 33.524 38.444) (width 0.2) (layer "F.Cu") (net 28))
 (segment (start 31.75 38.481) (end 33.487 38.481) (width 0.2) (layer "F.Cu") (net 28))
 (segment (start 21.971 37.495) (end 30.764 37.495) (width 0.2) (layer "F.Cu") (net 28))
 (segment (start 31.75 37.211) (end 33.487 37.211) (width 0.2) (layer "B.Cu") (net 29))
 (segment (start 21.971 35.495) (end 30.034 35.495) (width 0.2) (layer "B.Cu") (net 29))
 (segment (start 33.487 37.211) (end 33.524 37.174) (width 0.2) (layer "B.Cu") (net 29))
 (segment (start 30.034 35.495) (end 31.75 37.211) (width 0.2) (layer "B.Cu") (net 29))
 (segment (start 31.623 37.211) (end 33.487 37.211) (width 0.2) (layer "F.Cu") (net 30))
 (segment (start 33.487 37.211) (end 33.524 37.174) (width 0.2) (layer "F.Cu") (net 30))
 (segment (start 21.971 35.495) (end 29.907 35.495) (width 0.2) (layer "F.Cu") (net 30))
 (segment (start 29.907 35.495) (end 31.623 37.211) (width 0.2) (layer "F.Cu") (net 30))
 (segment (start 31.75 35.941) (end 33.487 35.941) (width 0.2) (layer "B.Cu") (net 31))
 (segment (start 21.971 33.495) (end 29.304 33.495) (width 0.2) (layer "B.Cu") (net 31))
 (segment (start 33.487 35.941) (end 33.524 35.904) (width 0.2) (layer "B.Cu") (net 31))
 (segment (start 29.304 33.495) (end 31.75 35.941) (width 0.2) (layer "B.Cu") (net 31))
 (segment (start 21.971 33.495) (end 29.431 33.495) (width 0.2) (layer "F.Cu") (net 32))
 (segment (start 31.877 35.941) (end 33.487 35.941) (width 0.2) (layer "F.Cu") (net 32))
 (segment (start 33.487 35.941) (end 33.524 35.904) (width 0.2) (layer "F.Cu") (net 32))
 (segment (start 29.431 33.495) (end 31.877 35.941) (width 0.2) (layer "F.Cu") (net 32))
 (segment (start 21.971 31.495) (end 28.574 31.495) (width 0.2) (layer "B.Cu") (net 33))
 (segment (start 31.75 34.671) (end 33.487 34.671) (width 0.2) (layer "B.Cu") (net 33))
 (segment (start 28.574 31.495) (end 31.75 34.671) (width 0.2) (layer "B.Cu") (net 33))
 (segment (start 33.487 34.671) (end 33.524 34.634) (width 0.2) (layer "B.Cu") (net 33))
 (segment (start 33.487 34.671) (end 33.524 34.634) (width 0.2) (layer "F.Cu") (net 34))
 (segment (start 28.574 31.495) (end 31.75 34.671) (width 0.2) (layer "F.Cu") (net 34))
 (segment (start 31.75 34.671) (end 33.487 34.671) (width 0.2) (layer "F.Cu") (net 34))
 (segment (start 21.971 31.495) (end 28.574 31.495) (width 0.2) (layer "F.Cu") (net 34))
 (segment (start 27.844 29.495) (end 31.75 33.401) (width 0.2) (layer "B.Cu") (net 35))
 (segment (start 21.971 29.495) (end 27.844 29.495) (width 0.2) (layer "B.Cu") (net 35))
 (segment (start 31.75 33.401) (end 33.487 33.401) (width 0.2) (layer "B.Cu") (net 35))
 (segment (start 33.487 33.401) (end 33.524 33.364) (width 0.2) (layer "B.Cu") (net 35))
 (segment (start 21.971 29.495) (end 27.971 29.495) (width 0.2) (layer "F.Cu") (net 36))
 (segment (start 33.487 33.401) (end 33.524 33.364) (width 0.2) (layer "F.Cu") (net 36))
 (segment (start 31.877 33.401) (end 33.487 33.401) (width 0.2) (layer "F.Cu") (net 36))
 (segment (start 27.971 29.495) (end 31.877 33.401) (width 0.2) (layer "F.Cu") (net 36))
 (segment (start 33.487 32.131) (end 33.524 32.094) (width 0.2) (layer "B.Cu") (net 37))
 (segment (start 21.971 27.495) (end 27.114 27.495) (width 0.2) (layer "B.Cu") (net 37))
 (segment (start 31.75 32.131) (end 33.487 32.131) (width 0.2) (layer "B.Cu") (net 37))
 (segment (start 27.114 27.495) (end 31.75 32.131) (width 0.2) (layer "B.Cu") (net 37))
 (segment (start 21.971 27.495) (end 27.114 27.495) (width 0.2) (layer "F.Cu") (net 38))
 (segment (start 31.75 32.131) (end 33.487 32.131) (width 0.2) (layer "F.Cu") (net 38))
 (segment (start 33.487 32.131) (end 33.524 32.094) (width 0.2) (layer "F.Cu") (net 38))
 (segment (start 27.114 27.495) (end 31.75 32.131) (width 0.2) (layer "F.Cu") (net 38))
 (segment (start 31.75 30.861) (end 33.487 30.861) (width 0.2) (layer "B.Cu") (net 39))
 (segment (start 26.384 25.495) (end 31.75 30.861) (width 0.2) (layer "B.Cu") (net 39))
 (segment (start 33.487 30.861) (end 33.524 30.824) (width 0.2) (layer "B.Cu") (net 39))
 (segment (start 21.971 25.495) (end 26.384 25.495) (width 0.2) (layer "B.Cu") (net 39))
 (segment (start 33.487 30.861) (end 33.524 30.824) (width 0.2) (layer "F.Cu") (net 40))
 (segment (start 31.75 30.861) (end 33.487 30.861) (width 0.2) (layer "F.Cu") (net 40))
 (segment (start 26.384 25.495) (end 31.75 30.861) (width 0.2) (layer "F.Cu") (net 40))
 (segment (start 21.971 25.495) (end 26.384 25.495) (width 0.2) (layer "F.Cu") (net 40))
 (segment (start 33.487 29.591) (end 33.524 29.554) (width 0.2) (layer "B.Cu") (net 41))
 (segment (start 31.75 29.591) (end 33.487 29.591) (width 0.2) (layer "B.Cu") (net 41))
 (segment (start 21.971 23.495) (end 25.654 23.495) (width 0.2) (layer "B.Cu") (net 41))
 (segment (start 25.654 23.495) (end 31.75 29.591) (width 0.2) (layer "B.Cu") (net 41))
 (segment (start 21.971 23.495) (end 25.781 23.495) (width 0.2) (layer "F.Cu") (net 42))
 (segment (start 31.877 29.591) (end 33.487 29.591) (width 0.2) (layer "F.Cu") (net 42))
 (segment (start 25.781 23.495) (end 31.877 29.591) (width 0.2) (layer "F.Cu") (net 42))
 (segment (start 33.487 29.591) (end 33.524 29.554) (width 0.2) (layer "F.Cu") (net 42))
 (segment (start 24.797 21.495) (end 31.623 28.321) (width 0.2) (layer "B.Cu") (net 43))
 (segment (start 21.971 21.495) (end 24.797 21.495) (width 0.2) (layer "B.Cu") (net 43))
 (segment (start 33.487 28.321) (end 33.524 28.284) (width 0.2) (layer "B.Cu") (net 43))
 (segment (start 31.623 28.321) (end 33.487 28.321) (width 0.2) (layer "B.Cu") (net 43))
 (segment (start 31.75 28.321) (end 33.487 28.321) (width 0.2) (layer "F.Cu") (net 44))
 (segment (start 21.971 21.495) (end 24.924 21.495) (width 0.2) (layer "F.Cu") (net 44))
 (segment (start 33.487 28.321) (end 33.524 28.284) (width 0.2) (layer "F.Cu") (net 44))
 (segment (start 24.924 21.495) (end 31.75 28.321) (width 0.2) (layer "F.Cu") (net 44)))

